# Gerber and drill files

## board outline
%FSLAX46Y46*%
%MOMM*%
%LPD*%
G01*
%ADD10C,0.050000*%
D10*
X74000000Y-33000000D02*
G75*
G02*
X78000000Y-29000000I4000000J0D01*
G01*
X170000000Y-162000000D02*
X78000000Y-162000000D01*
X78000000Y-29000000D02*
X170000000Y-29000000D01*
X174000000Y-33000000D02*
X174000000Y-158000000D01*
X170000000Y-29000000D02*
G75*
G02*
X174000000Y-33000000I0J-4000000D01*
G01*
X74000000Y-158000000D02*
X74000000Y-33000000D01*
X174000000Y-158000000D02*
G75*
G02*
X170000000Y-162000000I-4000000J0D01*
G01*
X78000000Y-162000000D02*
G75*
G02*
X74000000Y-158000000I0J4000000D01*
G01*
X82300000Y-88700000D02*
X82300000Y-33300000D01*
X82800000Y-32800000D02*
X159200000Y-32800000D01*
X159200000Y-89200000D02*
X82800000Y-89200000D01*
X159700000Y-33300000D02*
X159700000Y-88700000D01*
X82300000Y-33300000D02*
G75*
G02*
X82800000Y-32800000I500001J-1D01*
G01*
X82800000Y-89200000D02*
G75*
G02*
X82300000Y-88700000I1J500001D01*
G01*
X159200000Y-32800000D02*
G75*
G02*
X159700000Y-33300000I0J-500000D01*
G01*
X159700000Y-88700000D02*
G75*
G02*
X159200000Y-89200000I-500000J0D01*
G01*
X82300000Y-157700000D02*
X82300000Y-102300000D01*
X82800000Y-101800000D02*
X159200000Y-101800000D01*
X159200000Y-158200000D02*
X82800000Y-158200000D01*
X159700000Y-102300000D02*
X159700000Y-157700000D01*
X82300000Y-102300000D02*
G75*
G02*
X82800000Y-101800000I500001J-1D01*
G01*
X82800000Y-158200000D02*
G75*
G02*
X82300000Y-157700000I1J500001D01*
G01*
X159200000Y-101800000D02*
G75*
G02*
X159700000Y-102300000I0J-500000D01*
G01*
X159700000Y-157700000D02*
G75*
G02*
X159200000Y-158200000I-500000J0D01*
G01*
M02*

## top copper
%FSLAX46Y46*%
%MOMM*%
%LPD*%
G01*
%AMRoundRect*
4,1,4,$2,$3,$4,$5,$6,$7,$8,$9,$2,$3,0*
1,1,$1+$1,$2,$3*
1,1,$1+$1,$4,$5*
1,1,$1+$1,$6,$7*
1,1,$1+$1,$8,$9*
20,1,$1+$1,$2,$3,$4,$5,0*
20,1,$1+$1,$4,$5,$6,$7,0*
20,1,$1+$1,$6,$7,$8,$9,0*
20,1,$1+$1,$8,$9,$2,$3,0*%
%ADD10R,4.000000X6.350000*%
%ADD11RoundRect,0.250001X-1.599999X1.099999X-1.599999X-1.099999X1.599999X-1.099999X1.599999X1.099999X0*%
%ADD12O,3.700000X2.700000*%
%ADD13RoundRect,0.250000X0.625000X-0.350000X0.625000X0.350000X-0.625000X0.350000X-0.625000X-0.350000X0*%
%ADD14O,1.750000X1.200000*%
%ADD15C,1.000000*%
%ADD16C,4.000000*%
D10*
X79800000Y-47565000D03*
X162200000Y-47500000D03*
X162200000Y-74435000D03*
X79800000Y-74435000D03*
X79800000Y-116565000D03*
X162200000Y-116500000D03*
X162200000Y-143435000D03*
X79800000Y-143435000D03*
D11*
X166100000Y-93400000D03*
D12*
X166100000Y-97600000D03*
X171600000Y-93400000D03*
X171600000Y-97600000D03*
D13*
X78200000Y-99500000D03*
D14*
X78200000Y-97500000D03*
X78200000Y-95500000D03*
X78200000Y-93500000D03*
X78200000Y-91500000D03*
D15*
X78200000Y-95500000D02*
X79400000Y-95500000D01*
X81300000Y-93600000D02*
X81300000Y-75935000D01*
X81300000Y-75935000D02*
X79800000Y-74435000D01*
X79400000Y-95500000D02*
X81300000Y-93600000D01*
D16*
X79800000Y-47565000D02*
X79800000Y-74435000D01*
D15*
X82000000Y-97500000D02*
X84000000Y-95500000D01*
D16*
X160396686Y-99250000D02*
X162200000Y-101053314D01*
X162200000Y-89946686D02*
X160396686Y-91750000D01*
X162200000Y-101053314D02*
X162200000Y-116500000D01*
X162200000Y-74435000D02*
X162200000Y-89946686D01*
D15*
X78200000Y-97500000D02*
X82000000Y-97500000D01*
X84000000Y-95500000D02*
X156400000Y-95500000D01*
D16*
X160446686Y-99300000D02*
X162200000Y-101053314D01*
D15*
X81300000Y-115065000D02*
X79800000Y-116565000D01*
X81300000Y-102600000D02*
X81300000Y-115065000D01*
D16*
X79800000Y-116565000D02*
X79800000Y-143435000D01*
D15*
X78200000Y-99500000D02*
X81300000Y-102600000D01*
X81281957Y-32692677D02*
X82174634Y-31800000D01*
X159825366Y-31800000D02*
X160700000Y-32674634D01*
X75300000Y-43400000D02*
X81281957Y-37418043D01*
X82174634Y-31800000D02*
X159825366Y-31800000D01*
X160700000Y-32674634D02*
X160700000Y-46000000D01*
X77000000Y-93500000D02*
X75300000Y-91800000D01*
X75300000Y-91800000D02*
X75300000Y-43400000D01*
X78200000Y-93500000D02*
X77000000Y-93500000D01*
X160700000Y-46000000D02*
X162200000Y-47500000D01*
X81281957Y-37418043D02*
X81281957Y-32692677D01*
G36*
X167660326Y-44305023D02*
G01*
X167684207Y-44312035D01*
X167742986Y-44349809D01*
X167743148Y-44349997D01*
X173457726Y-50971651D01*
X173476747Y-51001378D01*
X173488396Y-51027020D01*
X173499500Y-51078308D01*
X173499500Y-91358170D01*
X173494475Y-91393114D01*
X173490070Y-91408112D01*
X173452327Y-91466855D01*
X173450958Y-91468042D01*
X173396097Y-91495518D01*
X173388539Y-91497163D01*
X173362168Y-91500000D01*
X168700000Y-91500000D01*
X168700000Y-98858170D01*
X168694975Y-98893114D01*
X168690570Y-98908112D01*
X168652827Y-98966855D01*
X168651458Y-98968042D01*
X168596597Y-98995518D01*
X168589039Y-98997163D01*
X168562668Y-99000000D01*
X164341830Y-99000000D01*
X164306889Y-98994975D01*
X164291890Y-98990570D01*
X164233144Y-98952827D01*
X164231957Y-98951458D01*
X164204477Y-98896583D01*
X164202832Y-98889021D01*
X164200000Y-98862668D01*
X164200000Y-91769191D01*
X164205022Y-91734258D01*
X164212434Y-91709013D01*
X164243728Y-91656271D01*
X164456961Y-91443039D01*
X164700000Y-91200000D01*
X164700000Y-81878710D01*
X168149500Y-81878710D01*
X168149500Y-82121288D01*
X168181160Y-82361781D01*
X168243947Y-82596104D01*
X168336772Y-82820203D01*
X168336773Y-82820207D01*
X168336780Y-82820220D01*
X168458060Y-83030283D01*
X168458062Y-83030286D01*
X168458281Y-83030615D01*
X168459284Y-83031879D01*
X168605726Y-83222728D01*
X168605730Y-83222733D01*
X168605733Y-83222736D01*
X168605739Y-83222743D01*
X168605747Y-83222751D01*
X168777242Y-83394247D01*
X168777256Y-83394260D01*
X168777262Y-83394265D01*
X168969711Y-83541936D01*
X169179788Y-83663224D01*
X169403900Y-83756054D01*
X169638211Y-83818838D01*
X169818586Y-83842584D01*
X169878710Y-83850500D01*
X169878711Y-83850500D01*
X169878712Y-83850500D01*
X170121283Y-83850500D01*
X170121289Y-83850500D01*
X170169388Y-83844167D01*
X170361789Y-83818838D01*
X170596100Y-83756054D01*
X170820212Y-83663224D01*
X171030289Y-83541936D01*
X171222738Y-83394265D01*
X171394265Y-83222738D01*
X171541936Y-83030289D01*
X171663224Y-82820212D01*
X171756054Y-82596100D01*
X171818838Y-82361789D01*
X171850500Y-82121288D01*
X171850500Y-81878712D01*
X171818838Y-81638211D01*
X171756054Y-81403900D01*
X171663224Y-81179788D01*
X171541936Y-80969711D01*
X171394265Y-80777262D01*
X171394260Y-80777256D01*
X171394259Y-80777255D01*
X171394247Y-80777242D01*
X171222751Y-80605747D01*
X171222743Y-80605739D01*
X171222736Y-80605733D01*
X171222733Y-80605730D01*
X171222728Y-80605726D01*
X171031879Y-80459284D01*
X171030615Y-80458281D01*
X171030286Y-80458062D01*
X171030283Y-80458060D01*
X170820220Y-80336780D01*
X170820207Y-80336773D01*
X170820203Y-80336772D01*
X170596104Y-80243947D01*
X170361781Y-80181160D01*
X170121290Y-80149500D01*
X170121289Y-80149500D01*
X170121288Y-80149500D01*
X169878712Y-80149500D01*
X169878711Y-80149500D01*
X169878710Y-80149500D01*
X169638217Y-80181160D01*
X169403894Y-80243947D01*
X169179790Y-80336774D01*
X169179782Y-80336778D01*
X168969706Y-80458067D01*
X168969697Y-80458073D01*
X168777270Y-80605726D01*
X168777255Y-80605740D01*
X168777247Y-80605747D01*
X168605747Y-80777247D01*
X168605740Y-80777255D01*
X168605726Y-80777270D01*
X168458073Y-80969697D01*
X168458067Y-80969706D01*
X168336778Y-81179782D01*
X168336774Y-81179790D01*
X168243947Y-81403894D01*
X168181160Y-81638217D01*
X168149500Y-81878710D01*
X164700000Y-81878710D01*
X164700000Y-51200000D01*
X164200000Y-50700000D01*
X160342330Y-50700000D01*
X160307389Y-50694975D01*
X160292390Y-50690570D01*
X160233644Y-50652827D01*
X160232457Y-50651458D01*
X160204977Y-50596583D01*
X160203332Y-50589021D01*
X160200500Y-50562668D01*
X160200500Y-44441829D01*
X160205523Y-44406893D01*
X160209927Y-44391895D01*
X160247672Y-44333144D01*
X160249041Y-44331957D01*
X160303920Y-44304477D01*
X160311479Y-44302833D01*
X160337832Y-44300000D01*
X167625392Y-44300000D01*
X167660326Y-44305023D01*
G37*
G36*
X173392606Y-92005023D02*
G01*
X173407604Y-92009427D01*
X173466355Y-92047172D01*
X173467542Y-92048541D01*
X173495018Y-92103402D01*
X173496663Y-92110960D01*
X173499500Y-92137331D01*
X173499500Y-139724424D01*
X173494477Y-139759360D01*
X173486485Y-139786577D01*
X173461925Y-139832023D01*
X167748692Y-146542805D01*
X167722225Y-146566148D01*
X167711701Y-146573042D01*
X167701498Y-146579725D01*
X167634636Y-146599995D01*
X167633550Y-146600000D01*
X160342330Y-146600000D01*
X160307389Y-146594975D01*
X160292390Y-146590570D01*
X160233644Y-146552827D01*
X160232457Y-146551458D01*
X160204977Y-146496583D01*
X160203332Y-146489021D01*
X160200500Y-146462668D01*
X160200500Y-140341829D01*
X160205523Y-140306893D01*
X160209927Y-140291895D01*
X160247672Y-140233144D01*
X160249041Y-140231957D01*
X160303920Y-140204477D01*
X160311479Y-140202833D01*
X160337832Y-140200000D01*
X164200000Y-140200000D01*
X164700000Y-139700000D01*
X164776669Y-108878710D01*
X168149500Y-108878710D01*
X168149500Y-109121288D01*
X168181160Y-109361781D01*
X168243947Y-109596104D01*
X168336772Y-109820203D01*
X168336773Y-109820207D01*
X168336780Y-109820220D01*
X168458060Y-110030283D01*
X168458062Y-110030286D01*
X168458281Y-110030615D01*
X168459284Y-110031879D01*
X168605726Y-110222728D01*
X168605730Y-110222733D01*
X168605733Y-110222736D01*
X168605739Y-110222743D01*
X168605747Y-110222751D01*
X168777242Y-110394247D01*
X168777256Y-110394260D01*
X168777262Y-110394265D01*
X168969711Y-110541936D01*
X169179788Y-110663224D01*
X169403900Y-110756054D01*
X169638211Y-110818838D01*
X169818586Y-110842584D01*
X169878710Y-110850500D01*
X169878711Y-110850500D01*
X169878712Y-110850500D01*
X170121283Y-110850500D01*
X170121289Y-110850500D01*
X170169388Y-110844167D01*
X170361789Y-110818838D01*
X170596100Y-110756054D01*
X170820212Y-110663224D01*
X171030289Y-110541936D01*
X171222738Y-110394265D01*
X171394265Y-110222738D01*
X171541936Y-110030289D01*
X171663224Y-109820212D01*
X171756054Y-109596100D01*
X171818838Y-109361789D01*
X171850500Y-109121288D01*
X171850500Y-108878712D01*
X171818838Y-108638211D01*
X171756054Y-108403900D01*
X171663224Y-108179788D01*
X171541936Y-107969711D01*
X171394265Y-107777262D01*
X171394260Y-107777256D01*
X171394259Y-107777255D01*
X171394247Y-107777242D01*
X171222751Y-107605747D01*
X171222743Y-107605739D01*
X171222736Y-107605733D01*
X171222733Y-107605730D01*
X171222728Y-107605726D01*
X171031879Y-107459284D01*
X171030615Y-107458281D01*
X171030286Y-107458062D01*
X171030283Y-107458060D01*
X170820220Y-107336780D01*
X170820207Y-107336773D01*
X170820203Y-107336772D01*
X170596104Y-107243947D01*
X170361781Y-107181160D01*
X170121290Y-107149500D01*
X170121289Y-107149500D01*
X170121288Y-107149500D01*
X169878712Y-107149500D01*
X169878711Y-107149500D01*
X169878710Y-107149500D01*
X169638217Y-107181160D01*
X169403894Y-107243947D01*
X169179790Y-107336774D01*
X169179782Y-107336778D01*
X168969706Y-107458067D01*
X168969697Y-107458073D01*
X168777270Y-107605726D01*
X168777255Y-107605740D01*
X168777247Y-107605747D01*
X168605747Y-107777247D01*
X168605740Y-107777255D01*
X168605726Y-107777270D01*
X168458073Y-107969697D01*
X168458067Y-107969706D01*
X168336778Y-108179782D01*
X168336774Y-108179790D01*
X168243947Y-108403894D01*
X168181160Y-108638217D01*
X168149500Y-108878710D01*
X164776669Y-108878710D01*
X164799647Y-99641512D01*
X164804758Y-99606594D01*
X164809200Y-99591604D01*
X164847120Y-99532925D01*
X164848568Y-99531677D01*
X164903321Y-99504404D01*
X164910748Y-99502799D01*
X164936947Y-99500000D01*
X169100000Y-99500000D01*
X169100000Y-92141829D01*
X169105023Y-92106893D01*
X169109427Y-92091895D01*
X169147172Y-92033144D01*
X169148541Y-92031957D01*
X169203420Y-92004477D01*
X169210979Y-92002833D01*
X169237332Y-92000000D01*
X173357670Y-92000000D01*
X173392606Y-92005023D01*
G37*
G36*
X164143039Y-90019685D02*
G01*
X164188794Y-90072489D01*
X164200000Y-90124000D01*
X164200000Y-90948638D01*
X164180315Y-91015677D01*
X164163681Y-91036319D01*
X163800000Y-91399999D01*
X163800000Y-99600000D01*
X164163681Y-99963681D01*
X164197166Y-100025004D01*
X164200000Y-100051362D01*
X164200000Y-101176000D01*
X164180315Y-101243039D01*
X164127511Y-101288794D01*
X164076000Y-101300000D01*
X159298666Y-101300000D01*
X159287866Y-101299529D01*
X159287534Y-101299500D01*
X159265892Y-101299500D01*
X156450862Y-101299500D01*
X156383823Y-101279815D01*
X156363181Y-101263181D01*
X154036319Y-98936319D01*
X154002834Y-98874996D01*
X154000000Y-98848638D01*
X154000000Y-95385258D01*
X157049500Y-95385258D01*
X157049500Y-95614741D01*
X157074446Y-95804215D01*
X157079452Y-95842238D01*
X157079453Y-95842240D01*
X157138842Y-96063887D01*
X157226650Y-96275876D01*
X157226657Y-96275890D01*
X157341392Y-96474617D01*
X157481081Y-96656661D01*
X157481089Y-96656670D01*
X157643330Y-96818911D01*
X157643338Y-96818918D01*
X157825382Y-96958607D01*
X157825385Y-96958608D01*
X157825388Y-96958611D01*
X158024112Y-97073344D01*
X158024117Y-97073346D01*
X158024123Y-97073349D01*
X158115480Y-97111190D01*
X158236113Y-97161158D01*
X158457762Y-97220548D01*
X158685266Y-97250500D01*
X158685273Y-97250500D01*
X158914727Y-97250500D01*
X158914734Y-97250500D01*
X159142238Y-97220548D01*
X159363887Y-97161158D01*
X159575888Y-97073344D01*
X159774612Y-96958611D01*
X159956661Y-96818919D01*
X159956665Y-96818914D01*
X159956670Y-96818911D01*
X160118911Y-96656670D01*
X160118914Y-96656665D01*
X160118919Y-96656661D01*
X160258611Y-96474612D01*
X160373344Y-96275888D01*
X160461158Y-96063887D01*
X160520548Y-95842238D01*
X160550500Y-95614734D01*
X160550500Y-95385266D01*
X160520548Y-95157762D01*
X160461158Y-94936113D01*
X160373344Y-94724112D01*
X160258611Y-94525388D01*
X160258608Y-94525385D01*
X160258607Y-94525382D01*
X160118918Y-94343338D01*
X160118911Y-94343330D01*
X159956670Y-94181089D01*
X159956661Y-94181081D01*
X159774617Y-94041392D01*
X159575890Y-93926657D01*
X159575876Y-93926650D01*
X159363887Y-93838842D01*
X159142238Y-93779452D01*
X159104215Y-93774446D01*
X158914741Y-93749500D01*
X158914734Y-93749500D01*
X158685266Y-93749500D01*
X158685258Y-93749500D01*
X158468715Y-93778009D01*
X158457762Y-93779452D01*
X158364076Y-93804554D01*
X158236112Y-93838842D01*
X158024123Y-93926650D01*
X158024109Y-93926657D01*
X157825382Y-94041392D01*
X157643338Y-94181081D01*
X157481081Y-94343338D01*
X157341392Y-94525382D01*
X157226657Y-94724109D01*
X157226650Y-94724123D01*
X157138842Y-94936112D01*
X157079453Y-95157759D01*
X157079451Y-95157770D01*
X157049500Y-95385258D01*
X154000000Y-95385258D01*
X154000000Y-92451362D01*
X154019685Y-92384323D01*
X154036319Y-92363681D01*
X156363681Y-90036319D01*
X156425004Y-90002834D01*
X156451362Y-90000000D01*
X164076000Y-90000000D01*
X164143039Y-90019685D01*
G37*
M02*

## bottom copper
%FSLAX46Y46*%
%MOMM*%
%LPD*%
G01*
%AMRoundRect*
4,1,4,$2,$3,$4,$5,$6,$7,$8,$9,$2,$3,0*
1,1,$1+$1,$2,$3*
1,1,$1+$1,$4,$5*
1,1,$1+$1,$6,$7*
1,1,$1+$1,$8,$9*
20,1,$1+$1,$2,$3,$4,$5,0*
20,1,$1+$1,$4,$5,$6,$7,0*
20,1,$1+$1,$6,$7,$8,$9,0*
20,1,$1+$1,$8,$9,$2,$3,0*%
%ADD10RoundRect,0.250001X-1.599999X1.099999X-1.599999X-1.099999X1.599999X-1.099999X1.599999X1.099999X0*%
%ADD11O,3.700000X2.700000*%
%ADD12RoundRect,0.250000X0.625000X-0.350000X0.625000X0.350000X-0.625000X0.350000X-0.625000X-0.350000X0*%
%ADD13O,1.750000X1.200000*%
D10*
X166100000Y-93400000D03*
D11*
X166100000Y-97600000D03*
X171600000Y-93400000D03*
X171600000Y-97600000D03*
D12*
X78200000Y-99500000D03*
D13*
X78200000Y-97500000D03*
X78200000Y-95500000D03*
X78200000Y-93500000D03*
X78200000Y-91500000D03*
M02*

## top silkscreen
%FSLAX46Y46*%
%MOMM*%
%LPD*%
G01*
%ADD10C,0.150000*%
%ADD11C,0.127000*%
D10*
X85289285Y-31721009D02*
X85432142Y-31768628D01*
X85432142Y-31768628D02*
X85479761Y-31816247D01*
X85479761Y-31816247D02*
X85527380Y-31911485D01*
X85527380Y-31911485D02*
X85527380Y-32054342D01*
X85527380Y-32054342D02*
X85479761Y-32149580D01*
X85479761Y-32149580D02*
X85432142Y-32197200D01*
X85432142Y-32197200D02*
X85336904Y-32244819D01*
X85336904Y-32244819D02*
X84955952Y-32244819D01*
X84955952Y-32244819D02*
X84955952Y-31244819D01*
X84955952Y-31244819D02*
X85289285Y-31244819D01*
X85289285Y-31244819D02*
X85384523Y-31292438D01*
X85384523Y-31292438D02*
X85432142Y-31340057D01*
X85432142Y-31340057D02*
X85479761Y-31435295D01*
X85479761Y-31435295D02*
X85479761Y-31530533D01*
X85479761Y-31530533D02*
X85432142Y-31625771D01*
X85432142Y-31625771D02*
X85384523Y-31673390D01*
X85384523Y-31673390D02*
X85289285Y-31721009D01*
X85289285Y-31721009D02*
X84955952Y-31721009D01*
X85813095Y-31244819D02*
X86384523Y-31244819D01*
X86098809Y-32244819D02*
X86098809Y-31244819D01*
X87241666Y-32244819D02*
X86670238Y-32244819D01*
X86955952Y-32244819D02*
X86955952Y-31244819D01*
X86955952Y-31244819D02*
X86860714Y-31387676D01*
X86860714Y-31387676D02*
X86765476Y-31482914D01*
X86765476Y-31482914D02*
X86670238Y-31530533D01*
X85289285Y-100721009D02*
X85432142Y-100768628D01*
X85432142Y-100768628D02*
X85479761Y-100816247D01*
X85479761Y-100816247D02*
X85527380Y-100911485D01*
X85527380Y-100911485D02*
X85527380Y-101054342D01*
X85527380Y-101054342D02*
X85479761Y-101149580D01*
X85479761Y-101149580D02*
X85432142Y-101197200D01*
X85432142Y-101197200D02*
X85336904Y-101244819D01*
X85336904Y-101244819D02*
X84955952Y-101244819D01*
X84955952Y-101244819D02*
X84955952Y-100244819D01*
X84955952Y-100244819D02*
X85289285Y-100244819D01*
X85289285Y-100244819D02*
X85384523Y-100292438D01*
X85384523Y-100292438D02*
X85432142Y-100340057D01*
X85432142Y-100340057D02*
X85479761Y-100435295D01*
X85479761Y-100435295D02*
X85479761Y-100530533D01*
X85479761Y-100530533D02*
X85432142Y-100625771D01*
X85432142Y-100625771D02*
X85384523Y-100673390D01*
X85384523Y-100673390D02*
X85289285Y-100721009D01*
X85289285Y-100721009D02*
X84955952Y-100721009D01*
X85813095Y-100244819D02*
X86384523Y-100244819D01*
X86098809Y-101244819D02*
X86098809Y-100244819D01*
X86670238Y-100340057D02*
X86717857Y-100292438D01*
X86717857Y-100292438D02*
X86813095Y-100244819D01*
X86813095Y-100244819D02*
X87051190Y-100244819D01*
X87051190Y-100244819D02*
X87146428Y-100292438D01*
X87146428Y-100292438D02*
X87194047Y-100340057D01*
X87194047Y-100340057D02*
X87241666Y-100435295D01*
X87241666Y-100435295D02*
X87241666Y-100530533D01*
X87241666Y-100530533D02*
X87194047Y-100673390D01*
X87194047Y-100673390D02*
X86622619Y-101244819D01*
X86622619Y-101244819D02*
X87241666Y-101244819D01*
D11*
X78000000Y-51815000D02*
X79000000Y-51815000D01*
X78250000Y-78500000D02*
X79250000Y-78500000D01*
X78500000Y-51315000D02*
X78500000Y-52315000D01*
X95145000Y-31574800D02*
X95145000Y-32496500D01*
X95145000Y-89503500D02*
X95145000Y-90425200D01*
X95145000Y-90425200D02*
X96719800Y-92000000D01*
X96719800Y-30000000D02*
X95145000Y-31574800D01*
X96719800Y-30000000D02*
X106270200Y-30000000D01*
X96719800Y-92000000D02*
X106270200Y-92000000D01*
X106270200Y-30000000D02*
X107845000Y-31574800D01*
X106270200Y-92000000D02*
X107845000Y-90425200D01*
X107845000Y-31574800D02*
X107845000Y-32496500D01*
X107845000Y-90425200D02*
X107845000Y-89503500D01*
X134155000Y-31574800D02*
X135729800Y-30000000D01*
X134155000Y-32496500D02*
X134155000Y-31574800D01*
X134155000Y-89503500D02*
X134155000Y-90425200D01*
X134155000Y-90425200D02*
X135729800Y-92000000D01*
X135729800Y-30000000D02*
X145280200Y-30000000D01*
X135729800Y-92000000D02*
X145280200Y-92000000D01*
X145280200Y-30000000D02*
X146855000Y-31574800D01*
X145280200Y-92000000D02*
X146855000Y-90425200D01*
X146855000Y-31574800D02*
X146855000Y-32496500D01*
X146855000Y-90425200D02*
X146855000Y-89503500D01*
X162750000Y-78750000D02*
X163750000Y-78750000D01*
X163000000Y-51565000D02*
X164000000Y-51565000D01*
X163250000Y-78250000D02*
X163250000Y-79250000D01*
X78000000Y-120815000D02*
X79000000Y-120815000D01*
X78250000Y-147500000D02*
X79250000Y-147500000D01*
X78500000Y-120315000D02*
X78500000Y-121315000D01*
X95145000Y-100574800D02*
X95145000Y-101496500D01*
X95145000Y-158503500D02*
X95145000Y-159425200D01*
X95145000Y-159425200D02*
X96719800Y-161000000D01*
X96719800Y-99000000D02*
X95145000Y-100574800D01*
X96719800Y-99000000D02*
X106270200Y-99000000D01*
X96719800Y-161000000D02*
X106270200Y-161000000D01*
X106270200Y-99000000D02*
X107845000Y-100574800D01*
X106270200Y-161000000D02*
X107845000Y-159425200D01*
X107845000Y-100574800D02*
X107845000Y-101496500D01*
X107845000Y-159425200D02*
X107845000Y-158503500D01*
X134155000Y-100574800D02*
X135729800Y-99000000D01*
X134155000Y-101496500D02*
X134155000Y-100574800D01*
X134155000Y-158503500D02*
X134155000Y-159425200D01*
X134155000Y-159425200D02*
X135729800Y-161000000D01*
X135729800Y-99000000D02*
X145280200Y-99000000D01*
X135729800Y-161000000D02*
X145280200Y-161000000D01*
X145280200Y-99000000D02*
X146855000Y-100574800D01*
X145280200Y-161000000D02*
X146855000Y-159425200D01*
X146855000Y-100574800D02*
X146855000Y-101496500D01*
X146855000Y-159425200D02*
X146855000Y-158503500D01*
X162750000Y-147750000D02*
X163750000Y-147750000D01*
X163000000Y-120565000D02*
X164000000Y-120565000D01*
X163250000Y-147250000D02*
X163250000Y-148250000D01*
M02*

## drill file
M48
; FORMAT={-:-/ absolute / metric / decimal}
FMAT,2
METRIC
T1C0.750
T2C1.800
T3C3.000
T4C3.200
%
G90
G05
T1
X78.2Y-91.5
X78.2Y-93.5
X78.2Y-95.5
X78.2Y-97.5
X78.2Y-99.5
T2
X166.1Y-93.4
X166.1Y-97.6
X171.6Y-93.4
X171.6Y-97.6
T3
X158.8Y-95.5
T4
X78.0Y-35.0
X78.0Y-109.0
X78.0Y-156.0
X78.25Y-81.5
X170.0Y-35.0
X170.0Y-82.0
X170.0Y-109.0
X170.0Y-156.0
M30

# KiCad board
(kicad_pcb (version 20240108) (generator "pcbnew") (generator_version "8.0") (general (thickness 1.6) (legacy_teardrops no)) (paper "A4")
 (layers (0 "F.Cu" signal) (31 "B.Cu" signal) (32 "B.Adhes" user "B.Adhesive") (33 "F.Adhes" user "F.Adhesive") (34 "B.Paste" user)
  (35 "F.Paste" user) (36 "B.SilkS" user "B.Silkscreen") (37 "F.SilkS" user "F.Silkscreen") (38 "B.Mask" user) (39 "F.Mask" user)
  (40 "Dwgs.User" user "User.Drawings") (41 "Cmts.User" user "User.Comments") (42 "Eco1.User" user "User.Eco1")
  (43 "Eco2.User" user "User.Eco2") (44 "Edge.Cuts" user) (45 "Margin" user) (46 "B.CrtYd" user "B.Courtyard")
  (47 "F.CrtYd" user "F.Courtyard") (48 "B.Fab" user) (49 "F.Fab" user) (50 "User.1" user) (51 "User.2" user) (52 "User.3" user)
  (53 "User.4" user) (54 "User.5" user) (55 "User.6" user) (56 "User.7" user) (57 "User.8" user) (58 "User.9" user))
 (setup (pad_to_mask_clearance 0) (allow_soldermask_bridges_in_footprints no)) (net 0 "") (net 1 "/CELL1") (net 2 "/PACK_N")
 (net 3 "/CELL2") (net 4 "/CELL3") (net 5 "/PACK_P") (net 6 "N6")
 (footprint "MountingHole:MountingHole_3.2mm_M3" (layer "F.Cu") (at 78.25 81.5)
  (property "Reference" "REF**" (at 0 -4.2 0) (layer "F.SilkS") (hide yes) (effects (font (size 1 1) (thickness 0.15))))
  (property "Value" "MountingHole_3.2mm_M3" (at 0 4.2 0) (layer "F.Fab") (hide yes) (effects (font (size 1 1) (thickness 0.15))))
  (pad "" np_thru_hole circle (at 0 0) (size 3.2 3.2) (drill 3.2) (layers "F&B.Cu" "*.Mask")))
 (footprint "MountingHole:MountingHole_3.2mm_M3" (layer "F.Cu") (at 78 156)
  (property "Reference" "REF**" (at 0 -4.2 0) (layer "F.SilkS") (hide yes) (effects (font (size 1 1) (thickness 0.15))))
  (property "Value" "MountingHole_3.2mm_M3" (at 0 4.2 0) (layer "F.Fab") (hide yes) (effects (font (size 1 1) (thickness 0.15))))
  (pad "" np_thru_hole circle (at 0 0) (size 3.2 3.2) (drill 3.2) (layers "*.Cu" "*.Mask")))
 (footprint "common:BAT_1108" (layer "F.Cu") (at 121 61)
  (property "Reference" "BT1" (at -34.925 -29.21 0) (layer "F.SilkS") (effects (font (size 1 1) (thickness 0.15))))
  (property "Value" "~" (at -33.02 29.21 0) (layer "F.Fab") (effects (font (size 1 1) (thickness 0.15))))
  (fp_line (start -43 -9.185) (end -42 -9.185) (stroke (width 0.127) (type solid)) (layer "F.SilkS"))
  (fp_line (start -42.75 17.5) (end -41.75 17.5) (stroke (width 0.127) (type solid)) (layer "F.SilkS"))
  (fp_line (start -42.5 -9.685) (end -42.5 -8.685) (stroke (width 0.127) (type solid)) (layer "F.SilkS"))
  (fp_line (start -25.855 -29.4252) (end -25.855 -28.5035) (stroke (width 0.127) (type solid)) (layer "F.SilkS"))
  (fp_line (start -25.855 28.5035) (end -25.855 29.4252) (stroke (width 0.127) (type solid)) (layer "F.SilkS"))
  (fp_line (start -25.855 29.4252) (end -24.2802 31) (stroke (width 0.127) (type solid)) (layer "F.SilkS"))
  (fp_line (start -24.2802 -31) (end -25.855 -29.4252) (stroke (width 0.127) (type solid)) (layer "F.SilkS"))
  (fp_line (start -24.2802 -31) (end -14.7298 -31) (stroke (width 0.127) (type solid)) (layer "F.SilkS"))
  (fp_line (start -24.2802 31) (end -14.7298 31) (stroke (width 0.127) (type solid)) (layer "F.SilkS"))
  (fp_line (start -14.7298 -31) (end -13.155 -29.4252) (stroke (width 0.127) (type solid)) (layer "F.SilkS"))
  (fp_line (start -14.7298 31) (end -13.155 29.4252) (stroke (width 0.127) (type solid)) (layer "F.SilkS"))
  (fp_line (start -13.155 -29.4252) (end -13.155 -28.5035) (stroke (width 0.127) (type solid)) (layer "F.SilkS"))
  (fp_line (start -13.155 29.4252) (end -13.155 28.5035) (stroke (width 0.127) (type solid)) (layer "F.SilkS"))
  (fp_line (start 13.155 -29.4252) (end 14.7298 -31) (stroke (width 0.127) (type solid)) (layer "F.SilkS"))
  (fp_line (start 13.155 -28.5035) (end 13.155 -29.4252) (stroke (width 0.127) (type solid)) (layer "F.SilkS"))
  (fp_line (start 13.155 28.5035) (end 13.155 29.4252) (stroke (width 0.127) (type solid)) (layer "F.SilkS"))
  (fp_line (start 13.155 29.4252) (end 14.7298 31) (stroke (width 0.127) (type solid)) (layer "F.SilkS"))
  (fp_line (start 14.7298 -31) (end 24.2802 -31) (stroke (width 0.127) (type solid)) (layer "F.SilkS"))
  (fp_line (start 14.7298 31) (end 24.2802 31) (stroke (width 0.127) (type solid)) (layer "F.SilkS"))
  (fp_line (start 24.2802 -31) (end 25.855 -29.4252) (stroke (width 0.127) (type solid)) (layer "F.SilkS"))
  (fp_line (start 24.2802 31) (end 25.855 29.4252) (stroke (width 0.127) (type solid)) (layer "F.SilkS"))
  (fp_line (start 25.855 -29.4252) (end 25.855 -28.5035) (stroke (width 0.127) (type solid)) (layer "F.SilkS"))
  (fp_line (start 25.855 29.4252) (end 25.855 28.5035) (stroke (width 0.127) (type solid)) (layer "F.SilkS"))
  (fp_line (start 41.75 17.75) (end 42.75 17.75) (stroke (width 0.127) (type solid)) (layer "F.SilkS"))
  (fp_line (start 42 -9.435) (end 43 -9.435) (stroke (width 0.127) (type solid)) (layer "F.SilkS"))
  (fp_line (start 42.25 17.25) (end 42.25 18.25) (stroke (width 0.127) (type solid)) (layer "F.SilkS"))
  (fp_line (start -38.7 27.7) (end -38.7 -27.7) (stroke (width 0.05) (type solid)) (layer "Edge.Cuts"))
  (fp_line (start -38.2 -28.2) (end 38.2 -28.2) (stroke (width 0.05) (type solid)) (layer "Edge.Cuts"))
  (fp_line (start 38.2 28.2) (end -38.2 28.2) (stroke (width 0.05) (type solid)) (layer "Edge.Cuts"))
  (fp_line (start 38.7 -27.7) (end 38.7 27.7) (stroke (width 0.05) (type solid)) (layer "Edge.Cuts"))
  (fp_arc (start -38.7 -27.7) (mid -38.553553 -28.053553) (end -38.2 -28.2) (stroke (width 0.05) (type default)) (layer "Edge.Cuts"))
  (fp_arc (start -38.2 28.2) (mid -38.553553 28.053553) (end -38.7 27.7) (stroke (width 0.05) (type default)) (layer "Edge.Cuts"))
  (fp_arc (start 38.2 -28.2) (mid 38.553553 -28.053553) (end 38.7 -27.7) (stroke (width 0.05) (type default)) (layer "Edge.Cuts"))
  (fp_arc (start 38.7 27.7) (mid 38.553553 28.053553) (end 38.2 28.2) (stroke (width 0.05) (type default)) (layer "Edge.Cuts"))
  (pad "1" smd rect (at -41.2 -13.435) (size 4 6.35) (layers "F.Cu" "F.Paste" "F.Mask") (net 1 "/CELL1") (solder_mask_margin 0.102))
  (pad "2" smd rect (at 41.2 -13.5) (size 4 6.35) (layers "F.Cu" "F.Paste" "F.Mask") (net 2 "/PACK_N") (solder_mask_margin 0.102))
  (pad "3" smd rect (at 41.2 13.435) (size 4 6.35) (layers "F.Cu" "F.Paste" "F.Mask") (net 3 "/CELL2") (solder_mask_margin 0.102))
  (pad "4" smd rect (at -41.2 13.435) (size 4 6.35) (layers "F.Cu" "F.Paste" "F.Mask") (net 1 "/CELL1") (solder_mask_margin 0.102)))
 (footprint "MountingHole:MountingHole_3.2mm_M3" (layer "F.Cu") (at 170 156)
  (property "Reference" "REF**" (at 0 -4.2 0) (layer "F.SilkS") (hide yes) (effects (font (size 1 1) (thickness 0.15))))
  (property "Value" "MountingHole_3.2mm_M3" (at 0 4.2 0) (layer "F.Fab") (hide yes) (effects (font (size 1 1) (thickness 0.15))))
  (pad "" np_thru_hole circle (at 0 0) (size 3.2 3.2) (drill 3.2) (layers "F&B.Cu" "*.Mask")))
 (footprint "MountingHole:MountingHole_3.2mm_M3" (layer "F.Cu") (at 170 82)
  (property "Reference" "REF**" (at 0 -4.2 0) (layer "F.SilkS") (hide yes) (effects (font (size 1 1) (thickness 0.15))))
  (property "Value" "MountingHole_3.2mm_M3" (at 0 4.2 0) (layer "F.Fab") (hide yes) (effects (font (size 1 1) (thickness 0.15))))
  (pad "" np_thru_hole circle (at 0 0) (size 3.2 3.2) (drill 3.2) (layers "F&B.Cu" "*.Mask")))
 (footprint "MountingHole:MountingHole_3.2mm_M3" (layer "F.Cu") (at 78 35)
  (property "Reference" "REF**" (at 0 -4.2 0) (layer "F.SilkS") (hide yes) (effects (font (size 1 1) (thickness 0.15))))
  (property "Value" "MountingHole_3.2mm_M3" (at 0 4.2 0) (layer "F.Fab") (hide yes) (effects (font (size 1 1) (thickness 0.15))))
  (pad "" np_thru_hole circle (at 0 0) (size 3.2 3.2) (drill 3.2) (layers "F&B.Cu" "*.Mask")))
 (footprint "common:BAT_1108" (layer "F.Cu") (at 121 130)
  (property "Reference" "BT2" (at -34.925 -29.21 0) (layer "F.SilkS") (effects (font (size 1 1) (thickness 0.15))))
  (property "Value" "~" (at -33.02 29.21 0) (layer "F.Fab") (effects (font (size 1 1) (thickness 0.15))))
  (fp_line (start -43 -9.185) (end -42 -9.185) (stroke (width 0.127) (type solid)) (layer "F.SilkS"))
  (fp_line (start -42.75 17.5) (end -41.75 17.5) (stroke (width 0.127) (type solid)) (layer "F.SilkS"))
  (fp_line (start -42.5 -9.685) (end -42.5 -8.685) (stroke (width 0.127) (type solid)) (layer "F.SilkS"))
  (fp_line (start -25.855 -29.4252) (end -25.855 -28.5035) (stroke (width 0.127) (type solid)) (layer "F.SilkS"))
  (fp_line (start -25.855 28.5035) (end -25.855 29.4252) (stroke (width 0.127) (type solid)) (layer "F.SilkS"))
  (fp_line (start -25.855 29.4252) (end -24.2802 31) (stroke (width 0.127) (type solid)) (layer "F.SilkS"))
  (fp_line (start -24.2802 -31) (end -25.855 -29.4252) (stroke (width 0.127) (type solid)) (layer "F.SilkS"))
  (fp_line (start -24.2802 -31) (end -14.7298 -31) (stroke (width 0.127) (type solid)) (layer "F.SilkS"))
  (fp_line (start -24.2802 31) (end -14.7298 31) (stroke (width 0.127) (type solid)) (layer "F.SilkS"))
  (fp_line (start -14.7298 -31) (end -13.155 -29.4252) (stroke (width 0.127) (type solid)) (layer "F.SilkS"))
  (fp_line (start -14.7298 31) (end -13.155 29.4252) (stroke (width 0.127) (type solid)) (layer "F.SilkS"))
  (fp_line (start -13.155 -29.4252) (end -13.155 -28.5035) (stroke (width 0.127) (type solid)) (layer "F.SilkS"))
  (fp_line (start -13.155 29.4252) (end -13.155 28.5035) (stroke (width 0.127) (type solid)) (layer "F.SilkS"))
  (fp_line (start 13.155 -29.4252) (end 14.7298 -31) (stroke (width 0.127) (type solid)) (layer "F.SilkS"))
  (fp_line (start 13.155 -28.5035) (end 13.155 -29.4252) (stroke (width 0.127) (type solid)) (layer "F.SilkS"))
  (fp_line (start 13.155 28.5035) (end 13.155 29.4252) (stroke (width 0.127) (type solid)) (layer "F.SilkS"))
  (fp_line (start 13.155 29.4252) (end 14.7298 31) (stroke (width 0.127) (type solid)) (layer "F.SilkS"))
  (fp_line (start 14.7298 -31) (end 24.2802 -31) (stroke (width 0.127) (type solid)) (layer "F.SilkS"))
  (fp_line (start 14.7298 31) (end 24.2802 31) (stroke (width 0.127) (type solid)) (layer "F.SilkS"))
  (fp_line (start 24.2802 -31) (end 25.855 -29.4252) (stroke (width 0.127) (type solid)) (layer "F.SilkS"))
  (fp_line (start 24.2802 31) (end 25.855 29.4252) (stroke (width 0.127) (type solid)) (layer "F.SilkS"))
  (fp_line (start 25.855 -29.4252) (end 25.855 -28.5035) (stroke (width 0.127) (type solid)) (layer "F.SilkS"))
  (fp_line (start 25.855 29.4252) (end 25.855 28.5035) (stroke (width 0.127) (type solid)) (layer "F.SilkS"))
  (fp_line (start 41.75 17.75) (end 42.75 17.75) (stroke (width 0.127) (type solid)) (layer "F.SilkS"))
  (fp_line (start 42 -9.435) (end 43 -9.435) (stroke (width 0.127) (type solid)) (layer "F.SilkS"))
  (fp_line (start 42.25 17.25) (end 42.25 18.25) (stroke (width 0.127) (type solid)) (layer "F.SilkS"))
  (fp_line (start -38.7 27.7) (end -38.7 -27.7) (stroke (width 0.05) (type solid)) (layer "Edge.Cuts"))
  (fp_line (start -38.2 -28.2) (end 38.2 -28.2) (stroke (width 0.05) (type solid)) (layer "Edge.Cuts"))
  (fp_line (start 38.2 28.2) (end -38.2 28.2) (stroke (width 0.05) (type solid)) (layer "Edge.Cuts"))
  (fp_line (start 38.7 -27.7) (end 38.7 27.7) (stroke (width 0.05) (type solid)) (layer "Edge.Cuts"))
  (fp_arc (start -38.7 -27.7) (mid -38.553553 -28.053553) (end -38.2 -28.2) (stroke (width 0.05) (type default)) (layer "Edge.Cuts"))
  (fp_arc (start -38.2 28.2) (mid -38.553553 28.053553) (end -38.7 27.7) (stroke (width 0.05) (type default)) (layer "Edge.Cuts"))
  (fp_arc (start 38.2 -28.2) (mid 38.553553 -28.053553) (end 38.7 -27.7) (stroke (width 0.05) (type default)) (layer "Edge.Cuts"))
  (fp_arc (start 38.7 27.7) (mid 38.553553 28.053553) (end 38.2 28.2) (stroke (width 0.05) (type default)) (layer "Edge.Cuts"))
  (pad "1" smd rect (at -41.2 -13.435) (size 4 6.35) (layers "F.Cu" "F.Paste" "F.Mask") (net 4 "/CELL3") (solder_mask_margin 0.102))
  (pad "2" smd rect (at 41.2 -13.5) (size 4 6.35) (layers "F.Cu" "F.Paste" "F.Mask") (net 3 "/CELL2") (solder_mask_margin 0.102))
  (pad "3" smd rect (at 41.2 13.435) (size 4 6.35) (layers "F.Cu" "F.Paste" "F.Mask") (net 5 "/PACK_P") (solder_mask_margin 0.102))
  (pad "4" smd rect (at -41.2 13.435) (size 4 6.35) (layers "F.Cu" "F.Paste" "F.Mask") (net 4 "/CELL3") (solder_mask_margin 0.102)))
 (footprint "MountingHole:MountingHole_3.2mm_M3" (layer "F.Cu") (at 170 35)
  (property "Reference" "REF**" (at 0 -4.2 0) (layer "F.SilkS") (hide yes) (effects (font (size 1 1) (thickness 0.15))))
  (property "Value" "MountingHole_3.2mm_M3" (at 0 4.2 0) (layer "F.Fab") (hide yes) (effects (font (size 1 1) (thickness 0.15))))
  (pad "" np_thru_hole circle (at 0 0) (size 3.2 3.2) (drill 3.2) (layers "F&B.Cu" "*.Mask")))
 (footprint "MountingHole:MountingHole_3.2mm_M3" (layer "F.Cu") (at 78 109)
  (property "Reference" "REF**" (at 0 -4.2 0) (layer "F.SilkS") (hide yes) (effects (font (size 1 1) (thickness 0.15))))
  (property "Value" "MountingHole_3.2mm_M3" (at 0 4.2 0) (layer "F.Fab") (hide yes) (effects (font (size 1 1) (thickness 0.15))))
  (pad "" np_thru_hole circle (at 0 0) (size 3.2 3.2) (drill 3.2) (layers "F&B.Cu" "*.Mask")))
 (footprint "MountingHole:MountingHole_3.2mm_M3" (layer "F.Cu") (at 170 109)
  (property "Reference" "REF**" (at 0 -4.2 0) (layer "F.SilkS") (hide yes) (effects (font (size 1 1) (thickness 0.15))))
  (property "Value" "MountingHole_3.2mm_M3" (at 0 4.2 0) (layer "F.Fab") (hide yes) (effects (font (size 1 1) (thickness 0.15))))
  (pad "" np_thru_hole circle (at 0 0) (size 3.2 3.2) (drill 3.2) (layers "F&B.Cu" "*.Mask")))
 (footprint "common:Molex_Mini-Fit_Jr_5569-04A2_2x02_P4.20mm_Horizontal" (layer "B.Cu") (at 166.1 93.4 -90)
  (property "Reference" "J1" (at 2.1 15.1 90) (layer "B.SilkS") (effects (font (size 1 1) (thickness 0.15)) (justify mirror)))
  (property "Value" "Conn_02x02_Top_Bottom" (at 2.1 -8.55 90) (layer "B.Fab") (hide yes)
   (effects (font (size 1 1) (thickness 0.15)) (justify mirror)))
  (pad "" np_thru_hole circle (at 2.1 7.3 270) (size 3 3) (drill 3) (layers "*.Cu" "*.Mask"))
  (pad "1" thru_hole roundrect (at 0 0 270) (size 2.7 3.7) (drill 1.8) (layers "*.Cu" "*.Mask") (remove_unused_layers no)
   (roundrect_rratio 0.092593) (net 2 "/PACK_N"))
  (pad "2" thru_hole oval (at 4.2 0 270) (size 2.7 3.7) (drill 1.8) (layers "*.Cu" "*.Mask") (remove_unused_layers no) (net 2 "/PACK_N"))
  (pad "3" thru_hole oval (at 0 -5.5 270) (size 2.7 3.7) (drill 1.8) (layers "*.Cu" "*.Mask") (remove_unused_layers no) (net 5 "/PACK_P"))
  (pad "4" thru_hole oval (at 4.2 -5.5 270) (size 2.7 3.7) (drill 1.8) (layers "*.Cu" "*.Mask") (remove_unused_layers no) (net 5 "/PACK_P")))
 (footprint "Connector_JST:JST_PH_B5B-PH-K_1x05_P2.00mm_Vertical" (layer "B.Cu") (at 78.2 99.5 90)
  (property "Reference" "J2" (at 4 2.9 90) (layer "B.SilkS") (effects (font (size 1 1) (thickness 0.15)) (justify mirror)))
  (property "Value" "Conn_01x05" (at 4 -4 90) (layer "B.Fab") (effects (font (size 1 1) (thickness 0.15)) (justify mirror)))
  (pad "1" thru_hole roundrect (at 0 0 90) (size 1.2 1.75) (drill 0.75) (layers "*.Cu" "*.Mask") (remove_unused_layers no)
   (roundrect_rratio 0.208333) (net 4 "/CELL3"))
  (pad "2" thru_hole oval (at 2 0 90) (size 1.2 1.75) (drill 0.75) (layers "*.Cu" "*.Mask") (remove_unused_layers no) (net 3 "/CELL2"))
  (pad "3" thru_hole oval (at 4 0 90) (size 1.2 1.75) (drill 0.75) (layers "*.Cu" "*.Mask") (remove_unused_layers no) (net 1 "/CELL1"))
  (pad "4" thru_hole oval (at 6 0 90) (size 1.2 1.75) (drill 0.75) (layers "*.Cu" "*.Mask") (remove_unused_layers no) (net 2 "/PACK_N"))
  (pad "5" thru_hole oval (at 8 0 90) (size 1.2 1.75) (drill 0.75) (layers "*.Cu" "*.Mask") (remove_unused_layers no) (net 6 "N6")))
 (gr_arc (start 74 33) (mid 75.171573 30.171573) (end 78 29) (stroke (width 0.05) (type default)) (layer "Edge.Cuts"))
 (gr_line (start 170 162) (end 78 162) (stroke (width 0.05) (type default)) (layer "Edge.Cuts"))
 (gr_line (start 78 29) (end 170 29) (stroke (width 0.05) (type default)) (layer "Edge.Cuts"))
 (gr_line (start 174 33) (end 174 158) (stroke (width 0.05) (type default)) (layer "Edge.Cuts"))
 (gr_arc (start 170 29) (mid 172.828427 30.171573) (end 174 33) (stroke (width 0.05) (type default)) (layer "Edge.Cuts"))
 (gr_line (start 74 158) (end 74 33) (stroke (width 0.05) (type default)) (layer "Edge.Cuts"))
 (gr_arc (start 174 158) (mid 172.828427 160.828427) (end 170 162) (stroke (width 0.05) (type default)) (layer "Edge.Cuts"))
 (gr_arc (start 78 162) (mid 75.171573 160.828427) (end 74 158) (stroke (width 0.05) (type default)) (layer "Edge.Cuts"))
 (segment (start 78.2 95.5) (end 79.4 95.5) (width 1) (layer "F.Cu") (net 1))
 (segment (start 81.3 93.6) (end 81.3 75.935) (width 1) (layer "F.Cu") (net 1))
 (segment (start 81.3 75.935) (end 79.8 74.435) (width 1) (layer "F.Cu") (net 1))
 (segment (start 79.4 95.5) (end 81.3 93.6) (width 1) (layer "F.Cu") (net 1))
 (segment (start 79.8 47.565) (end 79.8 74.435) (width 4) (layer "F.Cu") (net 1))
 (segment (start 82 97.5) (end 84 95.5) (width 1) (layer "F.Cu") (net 3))
 (segment (start 160.396686 99.25) (end 162.2 101.053314) (width 4) (layer "F.Cu") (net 3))
 (segment (start 162.2 89.946686) (end 160.396686 91.75) (width 4) (layer "F.Cu") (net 3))
 (segment (start 162.2 101.053314) (end 162.2 116.5) (width 4) (layer "F.Cu") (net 3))
 (segment (start 162.2 74.435) (end 162.2 89.946686) (width 4) (layer "F.Cu") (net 3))
 (segment (start 78.2 97.5) (end 82 97.5) (width 1) (layer "F.Cu") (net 3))
 (segment (start 84 95.5) (end 156.4 95.5) (width 1) (layer "F.Cu") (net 3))
 (segment (start 160.446686 99.3) (end 162.2 101.053314) (width 4) (layer "F.Cu") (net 3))
 (segment (start 81.3 115.065) (end 79.8 116.565) (width 1) (layer "F.Cu") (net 4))
 (segment (start 81.3 102.6) (end 81.3 115.065) (width 1) (layer "F.Cu") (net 4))
 (segment (start 79.8 116.565) (end 79.8 143.435) (width 4) (layer "F.Cu") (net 4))
 (segment (start 78.2 99.5) (end 81.3 102.6) (width 1) (layer "F.Cu") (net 4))
 (segment (start 81.281957 32.692677) (end 82.174634 31.8) (width 1) (layer "F.Cu") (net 2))
 (segment (start 159.825366 31.8) (end 160.7 32.674634) (width 1) (layer "F.Cu") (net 2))
 (segment (start 75.3 43.4) (end 81.281957 37.418043) (width 1) (layer "F.Cu") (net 2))
 (segment (start 82.174634 31.8) (end 159.825366 31.8) (width 1) (layer "F.Cu") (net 2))
 (segment (start 160.7 32.674634) (end 160.7 46) (width 1) (layer "F.Cu") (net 2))
 (segment (start 77 93.5) (end 75.3 91.8) (width 1) (layer "F.Cu") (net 2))
 (segment (start 75.3 91.8) (end 75.3 43.4) (width 1) (layer "F.Cu") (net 2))
 (segment (start 78.2 93.5) (end 77 93.5) (width 1) (layer "F.Cu") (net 2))
 (segment (start 160.7 46) (end 162.2 47.5) (width 1) (layer "F.Cu") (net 2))
 (segment (start 81.281957 37.418043) (end 81.281957 32.692677) (width 1) (layer "F.Cu") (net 2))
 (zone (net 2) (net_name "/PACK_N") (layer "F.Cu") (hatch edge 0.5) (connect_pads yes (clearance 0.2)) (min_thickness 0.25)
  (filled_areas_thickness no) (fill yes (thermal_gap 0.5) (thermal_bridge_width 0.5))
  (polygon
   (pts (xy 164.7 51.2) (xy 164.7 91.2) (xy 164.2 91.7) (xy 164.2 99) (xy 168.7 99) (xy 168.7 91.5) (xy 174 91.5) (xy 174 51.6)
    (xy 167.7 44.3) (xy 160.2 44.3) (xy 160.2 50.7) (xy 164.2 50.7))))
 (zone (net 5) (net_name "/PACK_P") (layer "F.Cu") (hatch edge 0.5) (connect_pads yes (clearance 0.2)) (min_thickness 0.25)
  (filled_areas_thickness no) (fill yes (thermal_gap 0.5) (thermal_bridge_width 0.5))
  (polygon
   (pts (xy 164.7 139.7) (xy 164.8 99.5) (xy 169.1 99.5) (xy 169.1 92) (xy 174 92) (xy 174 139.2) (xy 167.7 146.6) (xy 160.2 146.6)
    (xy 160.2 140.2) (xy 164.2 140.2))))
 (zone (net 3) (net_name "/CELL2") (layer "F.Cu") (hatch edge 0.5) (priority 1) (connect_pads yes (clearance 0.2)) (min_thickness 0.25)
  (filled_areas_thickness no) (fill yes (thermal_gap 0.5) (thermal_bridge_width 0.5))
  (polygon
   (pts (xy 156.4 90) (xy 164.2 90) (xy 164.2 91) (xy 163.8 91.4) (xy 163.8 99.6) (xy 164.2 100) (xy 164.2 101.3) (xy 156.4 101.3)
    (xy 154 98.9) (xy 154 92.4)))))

